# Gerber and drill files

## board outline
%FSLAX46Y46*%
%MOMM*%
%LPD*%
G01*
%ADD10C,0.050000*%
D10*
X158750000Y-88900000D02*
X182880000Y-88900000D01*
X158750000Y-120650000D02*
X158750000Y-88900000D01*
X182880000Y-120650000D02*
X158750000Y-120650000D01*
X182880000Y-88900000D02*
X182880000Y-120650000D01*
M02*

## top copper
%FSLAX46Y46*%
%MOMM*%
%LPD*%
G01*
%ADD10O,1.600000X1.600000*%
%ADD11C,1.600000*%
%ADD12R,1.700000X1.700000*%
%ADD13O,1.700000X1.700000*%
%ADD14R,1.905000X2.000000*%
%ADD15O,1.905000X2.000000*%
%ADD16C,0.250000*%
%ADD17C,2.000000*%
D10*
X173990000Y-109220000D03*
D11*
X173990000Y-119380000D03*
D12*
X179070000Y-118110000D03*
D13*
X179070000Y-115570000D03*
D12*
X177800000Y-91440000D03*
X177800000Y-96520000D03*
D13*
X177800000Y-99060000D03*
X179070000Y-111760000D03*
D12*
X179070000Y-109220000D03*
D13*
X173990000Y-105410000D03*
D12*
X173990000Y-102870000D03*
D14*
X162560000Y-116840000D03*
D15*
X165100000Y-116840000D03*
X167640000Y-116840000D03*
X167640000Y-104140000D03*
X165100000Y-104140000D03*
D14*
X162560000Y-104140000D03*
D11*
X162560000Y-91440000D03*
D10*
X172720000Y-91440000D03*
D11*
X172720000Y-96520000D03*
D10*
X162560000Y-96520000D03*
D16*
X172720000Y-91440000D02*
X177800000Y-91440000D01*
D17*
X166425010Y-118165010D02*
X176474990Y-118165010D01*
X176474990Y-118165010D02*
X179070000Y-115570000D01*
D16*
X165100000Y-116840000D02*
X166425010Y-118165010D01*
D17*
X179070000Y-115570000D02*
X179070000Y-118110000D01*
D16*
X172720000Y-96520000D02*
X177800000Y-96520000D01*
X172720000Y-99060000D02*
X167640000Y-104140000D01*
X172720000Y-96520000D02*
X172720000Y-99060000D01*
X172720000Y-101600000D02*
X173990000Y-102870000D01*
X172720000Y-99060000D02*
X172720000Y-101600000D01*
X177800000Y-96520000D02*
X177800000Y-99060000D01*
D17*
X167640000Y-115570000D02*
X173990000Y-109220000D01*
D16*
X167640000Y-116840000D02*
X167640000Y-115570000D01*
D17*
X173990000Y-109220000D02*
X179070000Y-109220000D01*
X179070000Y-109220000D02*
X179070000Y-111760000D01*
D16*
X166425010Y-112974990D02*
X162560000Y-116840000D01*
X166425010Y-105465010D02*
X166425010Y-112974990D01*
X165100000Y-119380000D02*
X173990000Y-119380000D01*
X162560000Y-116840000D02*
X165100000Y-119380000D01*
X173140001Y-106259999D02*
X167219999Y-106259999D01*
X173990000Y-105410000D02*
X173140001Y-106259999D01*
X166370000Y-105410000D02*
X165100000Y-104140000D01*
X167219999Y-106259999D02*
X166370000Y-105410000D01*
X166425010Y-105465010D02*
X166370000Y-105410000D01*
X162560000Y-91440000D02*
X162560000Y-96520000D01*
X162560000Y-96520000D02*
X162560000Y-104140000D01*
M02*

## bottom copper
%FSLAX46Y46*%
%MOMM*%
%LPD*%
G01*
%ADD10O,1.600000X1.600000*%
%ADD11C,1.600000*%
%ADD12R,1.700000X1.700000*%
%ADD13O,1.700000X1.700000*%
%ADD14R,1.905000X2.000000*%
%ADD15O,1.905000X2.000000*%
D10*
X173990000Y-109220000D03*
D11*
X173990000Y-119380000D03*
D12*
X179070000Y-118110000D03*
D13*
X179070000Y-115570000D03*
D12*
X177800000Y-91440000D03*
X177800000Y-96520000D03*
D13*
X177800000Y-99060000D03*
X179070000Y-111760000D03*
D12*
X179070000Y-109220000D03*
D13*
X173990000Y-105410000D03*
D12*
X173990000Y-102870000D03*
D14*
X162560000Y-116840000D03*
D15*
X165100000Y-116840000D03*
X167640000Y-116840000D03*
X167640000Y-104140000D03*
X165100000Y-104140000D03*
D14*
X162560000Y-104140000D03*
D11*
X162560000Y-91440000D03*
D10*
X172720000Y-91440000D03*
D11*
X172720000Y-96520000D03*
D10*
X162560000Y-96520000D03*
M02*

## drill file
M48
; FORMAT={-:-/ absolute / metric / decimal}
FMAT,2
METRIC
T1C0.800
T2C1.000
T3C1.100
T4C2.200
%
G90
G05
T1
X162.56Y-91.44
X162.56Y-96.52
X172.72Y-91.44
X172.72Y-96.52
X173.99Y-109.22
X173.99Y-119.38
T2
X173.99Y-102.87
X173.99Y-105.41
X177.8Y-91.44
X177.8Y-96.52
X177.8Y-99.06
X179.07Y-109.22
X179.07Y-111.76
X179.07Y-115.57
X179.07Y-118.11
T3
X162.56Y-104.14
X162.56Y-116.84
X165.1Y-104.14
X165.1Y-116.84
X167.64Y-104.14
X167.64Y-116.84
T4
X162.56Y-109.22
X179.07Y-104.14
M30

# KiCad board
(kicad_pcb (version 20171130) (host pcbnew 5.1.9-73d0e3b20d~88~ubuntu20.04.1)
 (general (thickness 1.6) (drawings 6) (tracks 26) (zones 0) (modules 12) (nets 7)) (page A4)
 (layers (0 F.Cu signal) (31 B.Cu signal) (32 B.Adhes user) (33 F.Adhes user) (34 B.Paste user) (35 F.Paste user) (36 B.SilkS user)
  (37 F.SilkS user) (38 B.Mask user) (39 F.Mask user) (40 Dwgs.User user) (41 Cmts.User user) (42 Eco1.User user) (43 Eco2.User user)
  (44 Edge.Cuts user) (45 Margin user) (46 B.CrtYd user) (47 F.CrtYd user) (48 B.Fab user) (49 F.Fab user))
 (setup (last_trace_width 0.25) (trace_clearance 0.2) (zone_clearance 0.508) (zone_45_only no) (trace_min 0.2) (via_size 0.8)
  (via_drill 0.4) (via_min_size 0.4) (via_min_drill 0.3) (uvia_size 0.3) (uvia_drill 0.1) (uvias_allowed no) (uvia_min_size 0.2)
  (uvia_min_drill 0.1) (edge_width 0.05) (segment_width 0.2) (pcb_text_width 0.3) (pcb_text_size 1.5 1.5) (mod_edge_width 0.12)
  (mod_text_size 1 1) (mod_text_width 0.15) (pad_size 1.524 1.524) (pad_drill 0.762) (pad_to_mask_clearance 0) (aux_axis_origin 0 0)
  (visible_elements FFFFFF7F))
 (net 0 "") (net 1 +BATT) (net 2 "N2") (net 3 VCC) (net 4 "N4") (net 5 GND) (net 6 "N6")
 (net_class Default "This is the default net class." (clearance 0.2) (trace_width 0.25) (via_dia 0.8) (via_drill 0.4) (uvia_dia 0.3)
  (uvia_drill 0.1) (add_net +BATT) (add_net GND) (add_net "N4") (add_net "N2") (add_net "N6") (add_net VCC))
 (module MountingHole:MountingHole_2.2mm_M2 (layer F.Cu) (at 162.56 109.22)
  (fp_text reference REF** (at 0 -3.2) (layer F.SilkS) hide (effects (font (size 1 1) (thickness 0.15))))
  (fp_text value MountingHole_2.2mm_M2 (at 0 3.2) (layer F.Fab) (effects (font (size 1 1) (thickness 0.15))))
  (pad 1 np_thru_hole circle (at 0 0) (size 2.2 2.2) (drill 2.2) (layers *.Cu *.Mask)))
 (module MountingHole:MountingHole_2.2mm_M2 (layer F.Cu) (at 179.07 104.14)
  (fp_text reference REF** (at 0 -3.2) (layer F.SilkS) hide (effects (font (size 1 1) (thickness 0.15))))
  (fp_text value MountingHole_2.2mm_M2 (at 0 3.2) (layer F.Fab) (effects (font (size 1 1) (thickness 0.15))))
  (pad 1 np_thru_hole circle (at 0 0) (size 2.2 2.2) (drill 2.2) (layers *.Cu *.Mask)))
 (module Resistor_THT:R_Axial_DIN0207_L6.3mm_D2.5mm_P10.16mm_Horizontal (layer F.Cu) (at 173.99 119.38 90)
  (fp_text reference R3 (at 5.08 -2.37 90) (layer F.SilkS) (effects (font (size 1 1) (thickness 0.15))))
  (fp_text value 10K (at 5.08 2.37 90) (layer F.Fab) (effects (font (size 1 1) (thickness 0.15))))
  (pad 2 thru_hole oval (at 10.16 0 90) (size 1.6 1.6) (drill 0.8) (layers *.Cu *.Mask) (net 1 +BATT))
  (pad 1 thru_hole circle (at 0 0 90) (size 1.6 1.6) (drill 0.8) (layers *.Cu *.Mask) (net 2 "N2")))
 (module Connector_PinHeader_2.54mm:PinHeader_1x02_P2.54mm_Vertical (layer F.Cu) (at 179.07 118.11 180)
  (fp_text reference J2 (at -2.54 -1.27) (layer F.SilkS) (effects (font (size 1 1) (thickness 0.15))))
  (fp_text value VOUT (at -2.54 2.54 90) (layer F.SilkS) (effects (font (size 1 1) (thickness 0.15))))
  (pad 1 thru_hole rect (at 0 0 180) (size 1.7 1.7) (drill 1) (layers *.Cu *.Mask) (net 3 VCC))
  (pad 2 thru_hole oval (at 0 2.54 180) (size 1.7 1.7) (drill 1) (layers *.Cu *.Mask) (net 3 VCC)))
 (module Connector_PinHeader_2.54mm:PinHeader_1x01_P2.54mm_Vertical (layer F.Cu) (at 177.8 91.44)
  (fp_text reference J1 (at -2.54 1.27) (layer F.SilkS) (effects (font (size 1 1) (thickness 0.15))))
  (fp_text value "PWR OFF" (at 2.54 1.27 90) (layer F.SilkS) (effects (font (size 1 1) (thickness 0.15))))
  (pad 1 thru_hole rect (at 0 0) (size 1.7 1.7) (drill 1) (layers *.Cu *.Mask) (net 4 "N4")))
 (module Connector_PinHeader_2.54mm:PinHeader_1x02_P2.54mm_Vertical (layer F.Cu) (at 177.8 96.52)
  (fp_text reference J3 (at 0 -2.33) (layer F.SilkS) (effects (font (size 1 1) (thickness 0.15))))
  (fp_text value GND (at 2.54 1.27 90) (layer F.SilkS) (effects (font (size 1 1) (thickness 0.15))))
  (pad 1 thru_hole rect (at 0 0) (size 1.7 1.7) (drill 1) (layers *.Cu *.Mask) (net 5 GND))
  (pad 2 thru_hole oval (at 0 2.54) (size 1.7 1.7) (drill 1) (layers *.Cu *.Mask) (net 5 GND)))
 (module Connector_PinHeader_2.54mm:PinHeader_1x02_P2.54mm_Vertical (layer F.Cu) (at 179.07 109.22)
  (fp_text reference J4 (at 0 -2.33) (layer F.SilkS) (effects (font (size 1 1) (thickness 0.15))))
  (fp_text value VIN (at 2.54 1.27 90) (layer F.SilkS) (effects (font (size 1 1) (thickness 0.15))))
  (pad 2 thru_hole oval (at 0 2.54) (size 1.7 1.7) (drill 1) (layers *.Cu *.Mask) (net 1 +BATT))
  (pad 1 thru_hole rect (at 0 0) (size 1.7 1.7) (drill 1) (layers *.Cu *.Mask) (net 1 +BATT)))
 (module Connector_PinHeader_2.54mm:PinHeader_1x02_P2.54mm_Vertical (layer F.Cu) (at 173.99 102.87)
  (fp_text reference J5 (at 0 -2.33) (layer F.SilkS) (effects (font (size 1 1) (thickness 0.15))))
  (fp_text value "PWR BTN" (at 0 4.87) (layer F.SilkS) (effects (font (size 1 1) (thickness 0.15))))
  (pad 2 thru_hole oval (at 0 2.54) (size 1.7 1.7) (drill 1) (layers *.Cu *.Mask) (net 2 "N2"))
  (pad 1 thru_hole rect (at 0 0) (size 1.7 1.7) (drill 1) (layers *.Cu *.Mask) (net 5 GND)))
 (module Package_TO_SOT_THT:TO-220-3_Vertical (layer F.Cu) (at 162.56 116.84)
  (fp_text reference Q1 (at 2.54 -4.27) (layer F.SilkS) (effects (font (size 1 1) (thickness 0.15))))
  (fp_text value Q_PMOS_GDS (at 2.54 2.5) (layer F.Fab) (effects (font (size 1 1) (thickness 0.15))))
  (pad 1 thru_hole rect (at 0 0) (size 1.905 2) (drill 1.1) (layers *.Cu *.Mask) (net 2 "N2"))
  (pad 2 thru_hole oval (at 2.54 0) (size 1.905 2) (drill 1.1) (layers *.Cu *.Mask) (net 3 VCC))
  (pad 3 thru_hole oval (at 5.08 0) (size 1.905 2) (drill 1.1) (layers *.Cu *.Mask) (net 1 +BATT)))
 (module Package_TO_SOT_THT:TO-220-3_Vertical (layer F.Cu) (at 162.56 104.14)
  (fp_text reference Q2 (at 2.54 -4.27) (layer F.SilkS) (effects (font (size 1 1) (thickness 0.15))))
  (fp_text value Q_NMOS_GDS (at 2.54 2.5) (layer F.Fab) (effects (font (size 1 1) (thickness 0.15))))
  (pad 3 thru_hole oval (at 5.08 0) (size 1.905 2) (drill 1.1) (layers *.Cu *.Mask) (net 5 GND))
  (pad 2 thru_hole oval (at 2.54 0) (size 1.905 2) (drill 1.1) (layers *.Cu *.Mask) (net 2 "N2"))
  (pad 1 thru_hole rect (at 0 0) (size 1.905 2) (drill 1.1) (layers *.Cu *.Mask) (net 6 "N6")))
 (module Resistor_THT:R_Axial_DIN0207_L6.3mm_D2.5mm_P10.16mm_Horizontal (layer F.Cu) (at 162.56 91.44)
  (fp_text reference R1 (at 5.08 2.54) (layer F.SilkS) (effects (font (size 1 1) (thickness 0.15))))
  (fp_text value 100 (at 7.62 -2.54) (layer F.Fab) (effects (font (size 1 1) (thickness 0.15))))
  (pad 1 thru_hole circle (at 0 0) (size 1.6 1.6) (drill 0.8) (layers *.Cu *.Mask) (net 6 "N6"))
  (pad 2 thru_hole oval (at 10.16 0) (size 1.6 1.6) (drill 0.8) (layers *.Cu *.Mask) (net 4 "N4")))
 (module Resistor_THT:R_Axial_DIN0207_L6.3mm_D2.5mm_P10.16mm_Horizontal (layer F.Cu) (at 172.72 96.52 180)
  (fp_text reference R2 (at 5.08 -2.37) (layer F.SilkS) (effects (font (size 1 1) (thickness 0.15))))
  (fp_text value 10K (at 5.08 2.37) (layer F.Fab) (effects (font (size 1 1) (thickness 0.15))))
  (pad 1 thru_hole circle (at 0 0 180) (size 1.6 1.6) (drill 0.8) (layers *.Cu *.Mask) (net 5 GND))
  (pad 2 thru_hole oval (at 10.16 0 180) (size 1.6 1.6) (drill 0.8) (layers *.Cu *.Mask) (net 6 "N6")))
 (gr_line (start 158.75 88.9) (end 182.88 88.9) (layer Edge.Cuts) (width 0.05))
 (gr_line (start 158.75 120.65) (end 158.75 88.9) (layer Edge.Cuts) (width 0.05))
 (gr_line (start 182.88 120.65) (end 158.75 120.65) (layer Edge.Cuts) (width 0.05))
 (gr_line (start 182.88 88.9) (end 182.88 120.65) (layer Edge.Cuts) (width 0.05))
 (segment (start 172.72 91.44) (end 177.8 91.44) (width 0.25) (layer F.Cu) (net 4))
 (segment (start 166.42501 118.16501) (end 176.47499 118.16501) (width 2) (layer F.Cu) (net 3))
 (segment (start 176.47499 118.16501) (end 179.07 115.57) (width 2) (layer F.Cu) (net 3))
 (segment (start 165.1 116.84) (end 166.42501 118.16501) (width 0.25) (layer F.Cu) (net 3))
 (segment (start 179.07 115.57) (end 179.07 118.11) (width 2) (layer F.Cu) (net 3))
 (segment (start 172.72 96.52) (end 177.8 96.52) (width 0.25) (layer F.Cu) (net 5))
 (segment (start 172.72 99.06) (end 167.64 104.14) (width 0.25) (layer F.Cu) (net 5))
 (segment (start 172.72 96.52) (end 172.72 99.06) (width 0.25) (layer F.Cu) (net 5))
 (segment (start 172.72 101.6) (end 173.99 102.87) (width 0.25) (layer F.Cu) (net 5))
 (segment (start 172.72 99.06) (end 172.72 101.6) (width 0.25) (layer F.Cu) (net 5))
 (segment (start 177.8 96.52) (end 177.8 99.06) (width 0.25) (layer F.Cu) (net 5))
 (segment (start 167.64 115.57) (end 173.99 109.22) (width 2) (layer F.Cu) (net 1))
 (segment (start 167.64 116.84) (end 167.64 115.57) (width 0.25) (layer F.Cu) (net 1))
 (segment (start 173.99 109.22) (end 179.07 109.22) (width 2) (layer F.Cu) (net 1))
 (segment (start 179.07 109.22) (end 179.07 111.76) (width 2) (layer F.Cu) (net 1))
 (segment (start 166.42501 112.97499) (end 162.56 116.84) (width 0.25) (layer F.Cu) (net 2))
 (segment (start 166.42501 105.46501) (end 166.42501 112.97499) (width 0.25) (layer F.Cu) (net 2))
 (segment (start 165.1 119.38) (end 173.99 119.38) (width 0.25) (layer F.Cu) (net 2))
 (segment (start 162.56 116.84) (end 165.1 119.38) (width 0.25) (layer F.Cu) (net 2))
 (segment (start 173.140001 106.259999) (end 167.219999 106.259999) (width 0.25) (layer F.Cu) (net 2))
 (segment (start 173.99 105.41) (end 173.140001 106.259999) (width 0.25) (layer F.Cu) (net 2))
 (segment (start 166.37 105.41) (end 165.1 104.14) (width 0.25) (layer F.Cu) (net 2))
 (segment (start 167.219999 106.259999) (end 166.37 105.41) (width 0.25) (layer F.Cu) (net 2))
 (segment (start 166.42501 105.46501) (end 166.37 105.41) (width 0.25) (layer F.Cu) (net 2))
 (segment (start 162.56 91.44) (end 162.56 96.52) (width 0.25) (layer F.Cu) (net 6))
 (segment (start 162.56 96.52) (end 162.56 104.14) (width 0.25) (layer F.Cu) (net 6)))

